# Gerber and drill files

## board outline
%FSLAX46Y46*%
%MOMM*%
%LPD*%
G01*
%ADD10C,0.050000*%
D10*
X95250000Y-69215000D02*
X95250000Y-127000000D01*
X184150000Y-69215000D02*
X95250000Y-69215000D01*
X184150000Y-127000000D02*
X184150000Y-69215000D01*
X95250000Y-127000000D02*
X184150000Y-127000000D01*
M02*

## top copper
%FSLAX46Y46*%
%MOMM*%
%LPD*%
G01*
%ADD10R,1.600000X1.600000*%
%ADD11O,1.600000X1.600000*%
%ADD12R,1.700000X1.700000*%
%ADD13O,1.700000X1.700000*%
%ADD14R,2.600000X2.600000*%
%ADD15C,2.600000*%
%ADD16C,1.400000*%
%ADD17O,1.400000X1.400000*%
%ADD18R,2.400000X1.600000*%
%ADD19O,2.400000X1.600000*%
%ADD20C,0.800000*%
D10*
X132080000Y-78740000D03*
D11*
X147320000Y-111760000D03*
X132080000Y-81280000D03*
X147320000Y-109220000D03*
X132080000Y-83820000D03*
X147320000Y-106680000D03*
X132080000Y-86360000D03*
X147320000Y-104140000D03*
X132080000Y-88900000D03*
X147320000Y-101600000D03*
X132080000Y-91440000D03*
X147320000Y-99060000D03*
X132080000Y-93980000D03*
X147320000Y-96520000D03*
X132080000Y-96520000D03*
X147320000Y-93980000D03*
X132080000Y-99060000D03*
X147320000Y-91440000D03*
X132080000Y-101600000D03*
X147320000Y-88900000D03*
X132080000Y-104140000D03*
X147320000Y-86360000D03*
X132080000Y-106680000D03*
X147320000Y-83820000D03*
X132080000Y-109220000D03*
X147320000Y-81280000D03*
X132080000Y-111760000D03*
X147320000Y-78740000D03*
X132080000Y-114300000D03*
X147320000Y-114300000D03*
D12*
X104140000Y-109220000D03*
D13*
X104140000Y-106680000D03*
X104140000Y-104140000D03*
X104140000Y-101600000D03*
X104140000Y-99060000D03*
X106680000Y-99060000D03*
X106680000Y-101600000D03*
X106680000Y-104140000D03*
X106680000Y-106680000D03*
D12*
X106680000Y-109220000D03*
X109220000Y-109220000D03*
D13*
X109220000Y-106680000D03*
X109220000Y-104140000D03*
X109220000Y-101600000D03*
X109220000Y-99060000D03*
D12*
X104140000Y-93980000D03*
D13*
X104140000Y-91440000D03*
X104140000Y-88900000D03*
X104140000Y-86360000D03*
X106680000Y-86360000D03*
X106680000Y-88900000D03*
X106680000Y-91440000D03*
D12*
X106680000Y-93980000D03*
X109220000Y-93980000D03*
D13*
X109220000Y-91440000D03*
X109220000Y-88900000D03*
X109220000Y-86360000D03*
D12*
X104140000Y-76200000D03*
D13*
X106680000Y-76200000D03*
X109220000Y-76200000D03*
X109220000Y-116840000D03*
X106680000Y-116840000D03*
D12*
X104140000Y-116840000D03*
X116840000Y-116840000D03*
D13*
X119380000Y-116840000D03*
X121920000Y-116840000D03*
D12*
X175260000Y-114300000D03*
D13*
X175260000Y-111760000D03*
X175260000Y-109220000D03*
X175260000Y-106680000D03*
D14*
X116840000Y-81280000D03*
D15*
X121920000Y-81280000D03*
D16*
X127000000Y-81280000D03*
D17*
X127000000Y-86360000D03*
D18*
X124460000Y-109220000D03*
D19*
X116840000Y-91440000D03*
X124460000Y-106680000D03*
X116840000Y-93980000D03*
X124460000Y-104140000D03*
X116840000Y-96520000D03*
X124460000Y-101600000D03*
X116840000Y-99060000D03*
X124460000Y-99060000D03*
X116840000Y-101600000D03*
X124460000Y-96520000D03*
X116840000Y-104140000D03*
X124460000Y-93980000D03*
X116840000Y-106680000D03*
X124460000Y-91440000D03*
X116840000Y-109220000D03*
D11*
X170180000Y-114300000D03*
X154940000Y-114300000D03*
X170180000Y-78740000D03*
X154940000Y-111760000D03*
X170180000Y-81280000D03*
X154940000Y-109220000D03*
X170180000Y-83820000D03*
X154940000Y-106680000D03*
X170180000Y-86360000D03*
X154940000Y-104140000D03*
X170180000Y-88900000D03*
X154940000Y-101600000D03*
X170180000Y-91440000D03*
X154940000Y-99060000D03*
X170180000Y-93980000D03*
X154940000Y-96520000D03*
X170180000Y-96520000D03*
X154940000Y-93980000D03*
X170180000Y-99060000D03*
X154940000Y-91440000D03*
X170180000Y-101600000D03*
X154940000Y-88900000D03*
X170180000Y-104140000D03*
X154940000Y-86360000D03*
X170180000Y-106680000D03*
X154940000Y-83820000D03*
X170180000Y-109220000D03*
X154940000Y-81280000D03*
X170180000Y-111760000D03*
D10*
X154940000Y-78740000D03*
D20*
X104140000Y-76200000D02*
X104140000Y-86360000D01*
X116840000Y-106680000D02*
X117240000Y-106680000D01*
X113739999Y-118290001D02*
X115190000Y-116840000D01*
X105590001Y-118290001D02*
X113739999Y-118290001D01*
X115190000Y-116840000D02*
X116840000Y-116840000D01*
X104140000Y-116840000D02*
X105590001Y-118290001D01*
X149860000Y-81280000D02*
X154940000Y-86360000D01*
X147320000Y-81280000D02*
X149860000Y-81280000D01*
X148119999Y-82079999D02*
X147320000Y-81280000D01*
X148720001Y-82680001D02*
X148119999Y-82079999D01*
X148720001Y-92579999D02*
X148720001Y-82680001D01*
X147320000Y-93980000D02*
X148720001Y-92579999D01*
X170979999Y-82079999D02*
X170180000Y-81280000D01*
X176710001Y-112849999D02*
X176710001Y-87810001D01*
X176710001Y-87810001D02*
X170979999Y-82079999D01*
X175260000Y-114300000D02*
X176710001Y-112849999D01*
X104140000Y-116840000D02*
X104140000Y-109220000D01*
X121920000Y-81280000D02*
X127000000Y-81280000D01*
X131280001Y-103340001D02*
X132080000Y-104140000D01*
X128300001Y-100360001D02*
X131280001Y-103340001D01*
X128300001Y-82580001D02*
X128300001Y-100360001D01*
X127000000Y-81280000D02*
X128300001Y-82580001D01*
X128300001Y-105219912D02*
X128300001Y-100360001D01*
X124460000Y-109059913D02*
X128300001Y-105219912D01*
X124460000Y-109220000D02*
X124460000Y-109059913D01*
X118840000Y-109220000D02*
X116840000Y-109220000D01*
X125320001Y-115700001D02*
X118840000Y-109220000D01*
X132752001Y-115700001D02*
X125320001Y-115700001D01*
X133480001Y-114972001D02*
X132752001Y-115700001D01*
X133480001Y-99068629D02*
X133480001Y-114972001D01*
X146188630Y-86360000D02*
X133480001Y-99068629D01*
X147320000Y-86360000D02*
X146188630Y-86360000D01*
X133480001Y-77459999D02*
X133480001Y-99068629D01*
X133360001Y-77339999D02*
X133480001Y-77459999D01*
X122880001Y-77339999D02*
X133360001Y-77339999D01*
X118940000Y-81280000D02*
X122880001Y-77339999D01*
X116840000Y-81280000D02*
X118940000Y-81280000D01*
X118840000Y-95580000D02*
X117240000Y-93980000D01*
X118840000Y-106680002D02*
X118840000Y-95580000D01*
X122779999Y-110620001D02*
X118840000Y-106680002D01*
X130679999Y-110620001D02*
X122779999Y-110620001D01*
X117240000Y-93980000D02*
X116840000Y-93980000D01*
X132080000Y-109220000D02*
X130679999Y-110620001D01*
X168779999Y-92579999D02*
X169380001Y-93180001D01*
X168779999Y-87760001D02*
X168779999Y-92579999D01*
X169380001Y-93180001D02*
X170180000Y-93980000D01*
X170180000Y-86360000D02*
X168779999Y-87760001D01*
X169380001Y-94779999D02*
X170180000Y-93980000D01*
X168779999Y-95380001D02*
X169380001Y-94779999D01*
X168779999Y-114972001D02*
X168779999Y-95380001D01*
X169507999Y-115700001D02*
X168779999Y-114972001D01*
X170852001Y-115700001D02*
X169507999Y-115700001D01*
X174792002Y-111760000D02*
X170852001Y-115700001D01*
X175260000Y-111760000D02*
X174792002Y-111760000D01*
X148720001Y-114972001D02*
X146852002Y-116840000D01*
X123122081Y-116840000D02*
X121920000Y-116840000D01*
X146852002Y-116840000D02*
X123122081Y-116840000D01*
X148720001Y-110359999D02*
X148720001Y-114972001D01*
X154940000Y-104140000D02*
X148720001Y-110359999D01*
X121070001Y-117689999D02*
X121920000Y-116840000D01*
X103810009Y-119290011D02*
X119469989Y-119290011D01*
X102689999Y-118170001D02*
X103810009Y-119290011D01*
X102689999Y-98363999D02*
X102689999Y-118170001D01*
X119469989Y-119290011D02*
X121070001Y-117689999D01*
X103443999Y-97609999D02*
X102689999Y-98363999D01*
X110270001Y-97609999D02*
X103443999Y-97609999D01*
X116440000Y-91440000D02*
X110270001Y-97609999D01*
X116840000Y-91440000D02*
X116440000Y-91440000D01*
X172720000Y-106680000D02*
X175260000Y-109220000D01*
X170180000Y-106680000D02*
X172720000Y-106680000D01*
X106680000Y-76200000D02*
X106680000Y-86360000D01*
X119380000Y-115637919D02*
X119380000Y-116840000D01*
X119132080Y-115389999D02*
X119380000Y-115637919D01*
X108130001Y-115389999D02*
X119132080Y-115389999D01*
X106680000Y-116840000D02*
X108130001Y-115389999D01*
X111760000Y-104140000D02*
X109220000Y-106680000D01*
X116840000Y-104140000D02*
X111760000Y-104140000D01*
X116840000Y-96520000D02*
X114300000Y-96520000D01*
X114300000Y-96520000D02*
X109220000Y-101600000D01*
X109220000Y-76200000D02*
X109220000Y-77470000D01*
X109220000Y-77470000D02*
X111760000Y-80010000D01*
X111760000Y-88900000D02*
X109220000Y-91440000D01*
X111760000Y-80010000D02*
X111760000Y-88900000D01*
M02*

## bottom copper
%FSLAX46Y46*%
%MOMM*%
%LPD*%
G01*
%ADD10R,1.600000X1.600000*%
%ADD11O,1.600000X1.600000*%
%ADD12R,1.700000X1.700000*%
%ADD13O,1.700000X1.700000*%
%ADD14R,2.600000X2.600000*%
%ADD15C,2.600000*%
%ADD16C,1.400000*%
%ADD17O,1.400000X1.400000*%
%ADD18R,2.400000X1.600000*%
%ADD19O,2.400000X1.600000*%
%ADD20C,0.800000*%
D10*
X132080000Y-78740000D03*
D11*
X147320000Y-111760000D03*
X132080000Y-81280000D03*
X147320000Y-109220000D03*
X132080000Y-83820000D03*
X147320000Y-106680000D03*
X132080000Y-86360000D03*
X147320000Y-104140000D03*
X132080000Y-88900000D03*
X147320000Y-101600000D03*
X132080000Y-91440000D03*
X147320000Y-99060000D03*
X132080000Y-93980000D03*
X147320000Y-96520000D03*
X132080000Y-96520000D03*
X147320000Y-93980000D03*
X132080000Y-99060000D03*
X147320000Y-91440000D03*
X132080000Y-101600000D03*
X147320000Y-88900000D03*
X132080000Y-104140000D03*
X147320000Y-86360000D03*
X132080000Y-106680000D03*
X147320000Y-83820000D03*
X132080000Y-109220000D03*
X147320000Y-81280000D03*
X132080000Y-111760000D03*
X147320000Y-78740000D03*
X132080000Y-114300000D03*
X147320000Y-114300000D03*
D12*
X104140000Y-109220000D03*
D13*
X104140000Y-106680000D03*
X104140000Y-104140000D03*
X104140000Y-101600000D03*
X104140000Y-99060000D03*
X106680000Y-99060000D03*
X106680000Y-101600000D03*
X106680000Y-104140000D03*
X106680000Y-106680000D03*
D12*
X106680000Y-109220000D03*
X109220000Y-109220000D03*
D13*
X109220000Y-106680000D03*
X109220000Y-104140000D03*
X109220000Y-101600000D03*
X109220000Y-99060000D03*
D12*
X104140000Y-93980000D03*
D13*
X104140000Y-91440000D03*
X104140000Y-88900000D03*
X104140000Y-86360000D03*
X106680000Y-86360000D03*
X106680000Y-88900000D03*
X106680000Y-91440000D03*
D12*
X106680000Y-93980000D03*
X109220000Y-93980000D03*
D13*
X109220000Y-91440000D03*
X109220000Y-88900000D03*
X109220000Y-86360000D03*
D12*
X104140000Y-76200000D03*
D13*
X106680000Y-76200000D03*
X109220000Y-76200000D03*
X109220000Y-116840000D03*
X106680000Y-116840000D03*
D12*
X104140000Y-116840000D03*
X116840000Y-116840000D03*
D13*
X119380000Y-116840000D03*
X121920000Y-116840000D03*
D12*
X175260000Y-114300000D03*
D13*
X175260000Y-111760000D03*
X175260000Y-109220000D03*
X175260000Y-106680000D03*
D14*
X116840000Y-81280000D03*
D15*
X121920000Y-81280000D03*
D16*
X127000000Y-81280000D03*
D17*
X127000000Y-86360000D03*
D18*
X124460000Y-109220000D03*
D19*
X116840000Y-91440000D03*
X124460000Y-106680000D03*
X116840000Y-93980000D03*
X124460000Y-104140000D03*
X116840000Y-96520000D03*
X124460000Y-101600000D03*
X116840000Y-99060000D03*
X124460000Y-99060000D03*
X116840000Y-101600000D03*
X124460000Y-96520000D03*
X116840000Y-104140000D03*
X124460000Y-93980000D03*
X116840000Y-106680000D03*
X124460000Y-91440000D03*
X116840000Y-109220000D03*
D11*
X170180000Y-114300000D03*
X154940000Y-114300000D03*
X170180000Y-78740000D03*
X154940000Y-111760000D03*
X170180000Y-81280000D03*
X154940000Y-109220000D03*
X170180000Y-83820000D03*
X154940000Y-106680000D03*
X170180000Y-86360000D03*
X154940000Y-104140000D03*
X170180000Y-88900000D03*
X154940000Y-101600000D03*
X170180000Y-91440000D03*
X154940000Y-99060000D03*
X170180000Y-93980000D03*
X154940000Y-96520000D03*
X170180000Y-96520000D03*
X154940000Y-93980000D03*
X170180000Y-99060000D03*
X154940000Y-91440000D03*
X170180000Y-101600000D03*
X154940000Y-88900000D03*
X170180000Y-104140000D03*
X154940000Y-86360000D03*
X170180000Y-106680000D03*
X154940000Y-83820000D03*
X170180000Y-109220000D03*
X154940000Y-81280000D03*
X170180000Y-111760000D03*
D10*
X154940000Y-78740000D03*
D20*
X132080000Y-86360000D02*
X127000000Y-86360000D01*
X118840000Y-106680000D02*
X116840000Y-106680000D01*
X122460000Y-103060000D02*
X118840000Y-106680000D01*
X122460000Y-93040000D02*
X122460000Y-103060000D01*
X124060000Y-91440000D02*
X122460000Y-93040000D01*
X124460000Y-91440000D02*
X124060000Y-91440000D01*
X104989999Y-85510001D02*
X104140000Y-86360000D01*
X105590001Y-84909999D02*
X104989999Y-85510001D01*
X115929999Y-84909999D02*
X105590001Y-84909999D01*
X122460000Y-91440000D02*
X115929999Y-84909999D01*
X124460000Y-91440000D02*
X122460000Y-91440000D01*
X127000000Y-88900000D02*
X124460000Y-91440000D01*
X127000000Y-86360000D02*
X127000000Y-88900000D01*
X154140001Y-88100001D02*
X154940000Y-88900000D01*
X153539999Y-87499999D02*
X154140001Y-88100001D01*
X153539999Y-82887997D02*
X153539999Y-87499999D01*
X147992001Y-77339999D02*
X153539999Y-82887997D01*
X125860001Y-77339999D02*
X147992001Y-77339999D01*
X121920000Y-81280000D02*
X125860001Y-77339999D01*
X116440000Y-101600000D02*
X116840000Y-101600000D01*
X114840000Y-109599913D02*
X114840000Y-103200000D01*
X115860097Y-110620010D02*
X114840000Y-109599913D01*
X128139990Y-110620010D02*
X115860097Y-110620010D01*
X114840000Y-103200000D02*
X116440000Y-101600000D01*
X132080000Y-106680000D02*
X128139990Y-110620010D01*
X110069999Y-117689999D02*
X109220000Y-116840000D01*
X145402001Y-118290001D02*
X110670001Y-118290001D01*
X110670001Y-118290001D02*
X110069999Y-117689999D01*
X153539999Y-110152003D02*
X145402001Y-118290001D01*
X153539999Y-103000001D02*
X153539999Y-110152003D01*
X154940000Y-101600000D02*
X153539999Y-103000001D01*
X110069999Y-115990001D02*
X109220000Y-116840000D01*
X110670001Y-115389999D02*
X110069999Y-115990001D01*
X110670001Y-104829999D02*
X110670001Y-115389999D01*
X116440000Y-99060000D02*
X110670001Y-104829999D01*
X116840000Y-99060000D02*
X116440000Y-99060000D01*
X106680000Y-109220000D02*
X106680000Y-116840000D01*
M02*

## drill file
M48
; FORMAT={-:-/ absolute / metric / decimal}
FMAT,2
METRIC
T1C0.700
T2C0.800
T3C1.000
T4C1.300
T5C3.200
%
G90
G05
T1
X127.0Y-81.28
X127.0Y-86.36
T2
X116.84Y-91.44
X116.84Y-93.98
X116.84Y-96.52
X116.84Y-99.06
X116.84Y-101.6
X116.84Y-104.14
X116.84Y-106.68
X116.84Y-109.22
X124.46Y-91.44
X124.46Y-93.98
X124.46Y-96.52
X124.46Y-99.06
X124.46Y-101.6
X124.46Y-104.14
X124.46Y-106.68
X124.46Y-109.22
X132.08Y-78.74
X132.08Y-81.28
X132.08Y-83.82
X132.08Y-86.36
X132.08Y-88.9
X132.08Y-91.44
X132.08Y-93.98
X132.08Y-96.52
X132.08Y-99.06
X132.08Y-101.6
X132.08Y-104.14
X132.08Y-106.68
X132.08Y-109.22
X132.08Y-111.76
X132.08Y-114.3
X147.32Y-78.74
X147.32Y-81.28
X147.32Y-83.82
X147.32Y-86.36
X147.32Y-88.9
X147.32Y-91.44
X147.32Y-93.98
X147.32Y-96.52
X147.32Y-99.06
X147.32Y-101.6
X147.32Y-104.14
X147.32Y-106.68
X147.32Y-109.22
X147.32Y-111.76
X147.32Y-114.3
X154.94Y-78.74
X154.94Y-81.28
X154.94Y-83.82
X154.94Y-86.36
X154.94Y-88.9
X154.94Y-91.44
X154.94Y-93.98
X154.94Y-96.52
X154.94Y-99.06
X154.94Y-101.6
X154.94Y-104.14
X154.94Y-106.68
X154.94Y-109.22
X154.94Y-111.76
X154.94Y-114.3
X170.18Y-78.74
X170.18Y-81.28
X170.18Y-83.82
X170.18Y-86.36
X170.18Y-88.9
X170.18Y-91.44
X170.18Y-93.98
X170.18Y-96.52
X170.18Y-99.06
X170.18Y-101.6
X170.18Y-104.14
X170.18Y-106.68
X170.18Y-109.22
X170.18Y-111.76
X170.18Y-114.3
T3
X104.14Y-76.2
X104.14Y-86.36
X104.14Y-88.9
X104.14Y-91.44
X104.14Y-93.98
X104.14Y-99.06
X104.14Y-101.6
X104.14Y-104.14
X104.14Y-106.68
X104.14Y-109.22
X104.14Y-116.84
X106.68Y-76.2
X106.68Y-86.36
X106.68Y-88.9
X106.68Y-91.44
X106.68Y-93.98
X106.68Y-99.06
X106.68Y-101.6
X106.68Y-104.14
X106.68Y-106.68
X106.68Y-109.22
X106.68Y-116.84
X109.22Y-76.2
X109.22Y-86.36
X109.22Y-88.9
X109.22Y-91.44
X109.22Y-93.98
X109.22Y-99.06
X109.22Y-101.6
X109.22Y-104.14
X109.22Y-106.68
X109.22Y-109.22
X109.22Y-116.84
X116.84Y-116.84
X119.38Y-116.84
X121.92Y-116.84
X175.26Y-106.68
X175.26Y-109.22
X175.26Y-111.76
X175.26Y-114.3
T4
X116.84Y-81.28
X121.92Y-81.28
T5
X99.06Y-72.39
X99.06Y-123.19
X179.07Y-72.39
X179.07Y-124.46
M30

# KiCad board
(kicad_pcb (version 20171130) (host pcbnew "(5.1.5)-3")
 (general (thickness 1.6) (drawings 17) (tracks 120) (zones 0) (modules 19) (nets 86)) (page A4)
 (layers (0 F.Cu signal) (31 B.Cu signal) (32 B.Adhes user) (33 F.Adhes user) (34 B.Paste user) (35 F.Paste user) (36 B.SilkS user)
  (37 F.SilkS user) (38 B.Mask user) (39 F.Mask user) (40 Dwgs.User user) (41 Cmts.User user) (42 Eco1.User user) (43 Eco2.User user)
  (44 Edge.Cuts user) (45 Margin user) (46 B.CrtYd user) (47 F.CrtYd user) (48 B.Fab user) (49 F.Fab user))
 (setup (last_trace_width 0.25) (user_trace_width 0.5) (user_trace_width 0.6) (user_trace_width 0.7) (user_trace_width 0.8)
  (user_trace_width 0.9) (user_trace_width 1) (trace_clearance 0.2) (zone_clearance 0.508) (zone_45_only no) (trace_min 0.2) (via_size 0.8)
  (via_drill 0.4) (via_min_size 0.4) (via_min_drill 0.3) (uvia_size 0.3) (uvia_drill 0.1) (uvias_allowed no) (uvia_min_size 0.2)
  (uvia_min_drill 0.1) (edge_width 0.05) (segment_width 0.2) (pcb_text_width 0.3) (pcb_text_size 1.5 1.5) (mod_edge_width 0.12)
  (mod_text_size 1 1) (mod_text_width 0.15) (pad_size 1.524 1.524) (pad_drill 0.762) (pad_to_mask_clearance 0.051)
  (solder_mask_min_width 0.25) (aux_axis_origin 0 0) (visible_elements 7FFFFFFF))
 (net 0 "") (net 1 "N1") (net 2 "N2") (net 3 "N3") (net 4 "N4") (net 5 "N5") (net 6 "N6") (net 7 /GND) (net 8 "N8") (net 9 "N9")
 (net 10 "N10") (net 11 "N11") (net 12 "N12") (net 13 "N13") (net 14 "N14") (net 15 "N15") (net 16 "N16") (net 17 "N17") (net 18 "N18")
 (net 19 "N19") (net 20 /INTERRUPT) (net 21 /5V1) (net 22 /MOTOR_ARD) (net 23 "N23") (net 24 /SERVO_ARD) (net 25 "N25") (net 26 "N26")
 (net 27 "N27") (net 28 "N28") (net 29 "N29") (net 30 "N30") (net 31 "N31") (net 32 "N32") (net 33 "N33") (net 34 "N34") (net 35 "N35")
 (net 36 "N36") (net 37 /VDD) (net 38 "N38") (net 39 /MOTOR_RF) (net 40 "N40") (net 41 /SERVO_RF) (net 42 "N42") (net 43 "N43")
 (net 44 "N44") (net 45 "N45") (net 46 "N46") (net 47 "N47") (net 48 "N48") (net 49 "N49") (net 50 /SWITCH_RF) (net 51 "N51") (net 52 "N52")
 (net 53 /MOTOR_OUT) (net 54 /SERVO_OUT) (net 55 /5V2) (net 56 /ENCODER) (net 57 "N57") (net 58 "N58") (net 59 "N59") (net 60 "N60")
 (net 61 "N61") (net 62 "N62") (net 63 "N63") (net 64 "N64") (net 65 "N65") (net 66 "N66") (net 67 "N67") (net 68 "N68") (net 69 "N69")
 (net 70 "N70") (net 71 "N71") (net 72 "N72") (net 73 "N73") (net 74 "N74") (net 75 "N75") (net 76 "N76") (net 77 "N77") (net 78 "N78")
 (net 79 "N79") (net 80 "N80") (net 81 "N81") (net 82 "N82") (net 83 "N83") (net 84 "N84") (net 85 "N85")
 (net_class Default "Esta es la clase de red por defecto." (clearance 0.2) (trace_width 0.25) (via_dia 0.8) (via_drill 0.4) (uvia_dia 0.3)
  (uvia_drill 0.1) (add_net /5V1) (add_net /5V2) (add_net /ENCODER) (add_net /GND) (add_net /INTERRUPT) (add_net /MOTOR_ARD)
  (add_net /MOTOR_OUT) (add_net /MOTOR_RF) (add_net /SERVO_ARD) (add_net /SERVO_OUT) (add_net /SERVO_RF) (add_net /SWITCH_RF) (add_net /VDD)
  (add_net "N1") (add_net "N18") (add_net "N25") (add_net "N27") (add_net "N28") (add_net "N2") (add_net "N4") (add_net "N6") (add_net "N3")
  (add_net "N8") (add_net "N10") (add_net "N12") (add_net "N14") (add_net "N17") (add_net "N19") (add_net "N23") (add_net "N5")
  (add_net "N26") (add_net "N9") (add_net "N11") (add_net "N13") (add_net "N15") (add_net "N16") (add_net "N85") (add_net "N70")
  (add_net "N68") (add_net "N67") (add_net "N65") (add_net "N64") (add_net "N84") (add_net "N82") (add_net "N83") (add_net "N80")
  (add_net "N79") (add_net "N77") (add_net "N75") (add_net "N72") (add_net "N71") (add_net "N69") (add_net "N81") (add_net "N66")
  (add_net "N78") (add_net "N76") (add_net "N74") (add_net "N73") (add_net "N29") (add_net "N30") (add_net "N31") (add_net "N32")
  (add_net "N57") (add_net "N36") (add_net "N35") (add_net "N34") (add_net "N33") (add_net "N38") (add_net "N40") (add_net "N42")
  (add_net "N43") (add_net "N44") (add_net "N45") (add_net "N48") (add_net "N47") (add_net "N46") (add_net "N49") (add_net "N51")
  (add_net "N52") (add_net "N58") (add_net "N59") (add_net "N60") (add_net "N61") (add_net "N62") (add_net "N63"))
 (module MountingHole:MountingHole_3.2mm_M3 (layer F.Cu) (at 99.06 123.19)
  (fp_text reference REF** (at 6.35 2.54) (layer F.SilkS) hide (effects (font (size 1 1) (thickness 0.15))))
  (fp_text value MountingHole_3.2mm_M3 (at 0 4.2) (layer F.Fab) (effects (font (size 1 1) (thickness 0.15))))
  (pad 1 np_thru_hole circle (at 0 0) (size 3.2 3.2) (drill 3.2) (layers *.Cu *.Mask)))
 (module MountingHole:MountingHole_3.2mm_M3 (layer F.Cu) (at 99.06 72.39)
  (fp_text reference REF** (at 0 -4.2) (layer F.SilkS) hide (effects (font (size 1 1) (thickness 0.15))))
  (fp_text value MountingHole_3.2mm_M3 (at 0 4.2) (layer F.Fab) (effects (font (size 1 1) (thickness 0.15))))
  (pad 1 np_thru_hole circle (at 0 0) (size 3.2 3.2) (drill 3.2) (layers *.Cu *.Mask)))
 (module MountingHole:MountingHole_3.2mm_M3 (layer F.Cu) (at 179.07 72.39)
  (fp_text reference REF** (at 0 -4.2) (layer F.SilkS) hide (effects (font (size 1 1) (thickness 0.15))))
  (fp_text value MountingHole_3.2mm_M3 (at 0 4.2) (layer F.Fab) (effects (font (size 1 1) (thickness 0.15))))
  (pad 1 np_thru_hole circle (at 0 0) (size 3.2 3.2) (drill 3.2) (layers *.Cu *.Mask)))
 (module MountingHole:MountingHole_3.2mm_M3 (layer F.Cu) (at 179.07 124.46)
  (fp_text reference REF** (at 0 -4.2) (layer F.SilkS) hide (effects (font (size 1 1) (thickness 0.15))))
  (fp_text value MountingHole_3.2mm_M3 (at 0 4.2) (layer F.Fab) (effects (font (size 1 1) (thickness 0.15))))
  (pad 1 np_thru_hole circle (at 0 0) (size 3.2 3.2) (drill 3.2) (layers *.Cu *.Mask)))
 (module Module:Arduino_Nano (layer F.Cu) (at 132.08 78.74)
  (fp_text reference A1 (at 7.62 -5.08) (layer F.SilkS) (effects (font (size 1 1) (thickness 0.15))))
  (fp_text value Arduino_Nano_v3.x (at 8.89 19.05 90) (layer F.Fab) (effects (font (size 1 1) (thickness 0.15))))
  (pad 1 thru_hole rect (at 0 0) (size 1.6 1.6) (drill 0.8) (layers *.Cu *.Mask) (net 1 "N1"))
  (pad 17 thru_hole oval (at 15.24 33.02) (size 1.6 1.6) (drill 0.8) (layers *.Cu *.Mask) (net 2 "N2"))
  (pad 2 thru_hole oval (at 0 2.54) (size 1.6 1.6) (drill 0.8) (layers *.Cu *.Mask) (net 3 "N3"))
  (pad 18 thru_hole oval (at 15.24 30.48) (size 1.6 1.6) (drill 0.8) (layers *.Cu *.Mask) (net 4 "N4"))
  (pad 3 thru_hole oval (at 0 5.08) (size 1.6 1.6) (drill 0.8) (layers *.Cu *.Mask) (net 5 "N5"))
  (pad 19 thru_hole oval (at 15.24 27.94) (size 1.6 1.6) (drill 0.8) (layers *.Cu *.Mask) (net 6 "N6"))
  (pad 4 thru_hole oval (at 0 7.62) (size 1.6 1.6) (drill 0.8) (layers *.Cu *.Mask) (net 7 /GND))
  (pad 20 thru_hole oval (at 15.24 25.4) (size 1.6 1.6) (drill 0.8) (layers *.Cu *.Mask) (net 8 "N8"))
  (pad 5 thru_hole oval (at 0 10.16) (size 1.6 1.6) (drill 0.8) (layers *.Cu *.Mask) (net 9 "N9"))
  (pad 21 thru_hole oval (at 15.24 22.86) (size 1.6 1.6) (drill 0.8) (layers *.Cu *.Mask) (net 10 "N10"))
  (pad 6 thru_hole oval (at 0 12.7) (size 1.6 1.6) (drill 0.8) (layers *.Cu *.Mask) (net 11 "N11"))
  (pad 22 thru_hole oval (at 15.24 20.32) (size 1.6 1.6) (drill 0.8) (layers *.Cu *.Mask) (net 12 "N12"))
  (pad 7 thru_hole oval (at 0 15.24) (size 1.6 1.6) (drill 0.8) (layers *.Cu *.Mask) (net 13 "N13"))
  (pad 23 thru_hole oval (at 15.24 17.78) (size 1.6 1.6) (drill 0.8) (layers *.Cu *.Mask) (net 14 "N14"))
  (pad 8 thru_hole oval (at 0 17.78) (size 1.6 1.6) (drill 0.8) (layers *.Cu *.Mask) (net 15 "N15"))
  (pad 24 thru_hole oval (at 15.24 15.24) (size 1.6 1.6) (drill 0.8) (layers *.Cu *.Mask) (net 7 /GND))
  (pad 9 thru_hole oval (at 0 20.32) (size 1.6 1.6) (drill 0.8) (layers *.Cu *.Mask) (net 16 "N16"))
  (pad 25 thru_hole oval (at 15.24 12.7) (size 1.6 1.6) (drill 0.8) (layers *.Cu *.Mask) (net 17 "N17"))
  (pad 10 thru_hole oval (at 0 22.86) (size 1.6 1.6) (drill 0.8) (layers *.Cu *.Mask) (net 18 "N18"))
  (pad 26 thru_hole oval (at 15.24 10.16) (size 1.6 1.6) (drill 0.8) (layers *.Cu *.Mask) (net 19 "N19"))
  (pad 11 thru_hole oval (at 0 25.4) (size 1.6 1.6) (drill 0.8) (layers *.Cu *.Mask) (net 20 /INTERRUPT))
  (pad 27 thru_hole oval (at 15.24 7.62) (size 1.6 1.6) (drill 0.8) (layers *.Cu *.Mask) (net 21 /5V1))
  (pad 12 thru_hole oval (at 0 27.94) (size 1.6 1.6) (drill 0.8) (layers *.Cu *.Mask) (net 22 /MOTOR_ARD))
  (pad 28 thru_hole oval (at 15.24 5.08) (size 1.6 1.6) (drill 0.8) (layers *.Cu *.Mask) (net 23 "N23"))
  (pad 13 thru_hole oval (at 0 30.48) (size 1.6 1.6) (drill 0.8) (layers *.Cu *.Mask) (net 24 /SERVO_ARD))
  (pad 29 thru_hole oval (at 15.24 2.54) (size 1.6 1.6) (drill 0.8) (layers *.Cu *.Mask) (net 7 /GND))
  (pad 14 thru_hole oval (at 0 33.02) (size 1.6 1.6) (drill 0.8) (layers *.Cu *.Mask) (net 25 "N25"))
  (pad 30 thru_hole oval (at 15.24 0) (size 1.6 1.6) (drill 0.8) (layers *.Cu *.Mask) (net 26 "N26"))
  (pad 15 thru_hole oval (at 0 35.56) (size 1.6 1.6) (drill 0.8) (layers *.Cu *.Mask) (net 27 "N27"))
  (pad 16 thru_hole oval (at 15.24 35.56) (size 1.6 1.6) (drill 0.8) (layers *.Cu *.Mask) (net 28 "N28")))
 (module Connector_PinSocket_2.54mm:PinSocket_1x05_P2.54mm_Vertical (layer F.Cu) (at 104.14 109.22 180)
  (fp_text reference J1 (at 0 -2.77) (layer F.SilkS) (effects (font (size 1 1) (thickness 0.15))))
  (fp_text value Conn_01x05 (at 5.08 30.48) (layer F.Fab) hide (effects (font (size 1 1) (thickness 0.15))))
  (pad 1 thru_hole rect (at 0 0 180) (size 1.7 1.7) (drill 1) (layers *.Cu *.Mask) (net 7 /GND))
  (pad 2 thru_hole oval (at 0 2.54 180) (size 1.7 1.7) (drill 1) (layers *.Cu *.Mask) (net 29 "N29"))
  (pad 3 thru_hole oval (at 0 5.08 180) (size 1.7 1.7) (drill 1) (layers *.Cu *.Mask) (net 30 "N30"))
  (pad 4 thru_hole oval (at 0 7.62 180) (size 1.7 1.7) (drill 1) (layers *.Cu *.Mask) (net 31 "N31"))
  (pad 5 thru_hole oval (at 0 10.16 180) (size 1.7 1.7) (drill 1) (layers *.Cu *.Mask) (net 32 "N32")))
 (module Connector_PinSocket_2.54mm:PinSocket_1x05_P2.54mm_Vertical (layer F.Cu) (at 106.68 109.22 180)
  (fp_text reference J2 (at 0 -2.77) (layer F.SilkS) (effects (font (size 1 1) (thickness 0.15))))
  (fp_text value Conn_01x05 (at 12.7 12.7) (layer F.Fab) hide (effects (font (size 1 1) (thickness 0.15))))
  (pad 5 thru_hole oval (at 0 10.16 180) (size 1.7 1.7) (drill 1) (layers *.Cu *.Mask) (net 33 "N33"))
  (pad 4 thru_hole oval (at 0 7.62 180) (size 1.7 1.7) (drill 1) (layers *.Cu *.Mask) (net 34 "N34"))
  (pad 3 thru_hole oval (at 0 5.08 180) (size 1.7 1.7) (drill 1) (layers *.Cu *.Mask) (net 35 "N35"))
  (pad 2 thru_hole oval (at 0 2.54 180) (size 1.7 1.7) (drill 1) (layers *.Cu *.Mask) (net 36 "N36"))
  (pad 1 thru_hole rect (at 0 0 180) (size 1.7 1.7) (drill 1) (layers *.Cu *.Mask) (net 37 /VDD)))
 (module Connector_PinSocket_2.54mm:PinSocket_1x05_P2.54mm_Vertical (layer F.Cu) (at 109.22 109.22 180)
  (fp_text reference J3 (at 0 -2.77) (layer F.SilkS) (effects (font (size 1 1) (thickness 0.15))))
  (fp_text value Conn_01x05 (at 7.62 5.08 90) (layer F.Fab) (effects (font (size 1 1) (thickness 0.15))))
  (pad 1 thru_hole rect (at 0 0 180) (size 1.7 1.7) (drill 1) (layers *.Cu *.Mask) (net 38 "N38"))
  (pad 2 thru_hole oval (at 0 2.54 180) (size 1.7 1.7) (drill 1) (layers *.Cu *.Mask) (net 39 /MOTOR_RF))
  (pad 3 thru_hole oval (at 0 5.08 180) (size 1.7 1.7) (drill 1) (layers *.Cu *.Mask) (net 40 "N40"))
  (pad 4 thru_hole oval (at 0 7.62 180) (size 1.7 1.7) (drill 1) (layers *.Cu *.Mask) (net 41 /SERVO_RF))
  (pad 5 thru_hole oval (at 0 10.16 180) (size 1.7 1.7) (drill 1) (layers *.Cu *.Mask) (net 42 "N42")))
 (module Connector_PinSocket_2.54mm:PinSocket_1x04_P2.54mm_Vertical (layer F.Cu) (at 104.14 93.98 180)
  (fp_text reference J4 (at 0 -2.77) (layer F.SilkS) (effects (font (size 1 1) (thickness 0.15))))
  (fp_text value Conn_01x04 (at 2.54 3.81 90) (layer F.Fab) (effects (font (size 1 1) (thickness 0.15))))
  (pad 1 thru_hole rect (at 0 0 180) (size 1.7 1.7) (drill 1) (layers *.Cu *.Mask) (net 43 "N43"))
  (pad 2 thru_hole oval (at 0 2.54 180) (size 1.7 1.7) (drill 1) (layers *.Cu *.Mask) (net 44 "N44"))
  (pad 3 thru_hole oval (at 0 5.08 180) (size 1.7 1.7) (drill 1) (layers *.Cu *.Mask) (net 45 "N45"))
  (pad 4 thru_hole oval (at 0 7.62 180) (size 1.7 1.7) (drill 1) (layers *.Cu *.Mask) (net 7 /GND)))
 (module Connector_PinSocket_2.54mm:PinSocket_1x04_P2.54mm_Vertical (layer F.Cu) (at 106.68 93.98 180)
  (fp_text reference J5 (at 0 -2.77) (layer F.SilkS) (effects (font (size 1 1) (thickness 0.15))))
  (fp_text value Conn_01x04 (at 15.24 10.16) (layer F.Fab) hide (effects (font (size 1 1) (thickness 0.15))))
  (pad 4 thru_hole oval (at 0 7.62 180) (size 1.7 1.7) (drill 1) (layers *.Cu *.Mask) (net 37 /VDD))
  (pad 3 thru_hole oval (at 0 5.08 180) (size 1.7 1.7) (drill 1) (layers *.Cu *.Mask) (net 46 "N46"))
  (pad 2 thru_hole oval (at 0 2.54 180) (size 1.7 1.7) (drill 1) (layers *.Cu *.Mask) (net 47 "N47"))
  (pad 1 thru_hole rect (at 0 0 180) (size 1.7 1.7) (drill 1) (layers *.Cu *.Mask) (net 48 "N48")))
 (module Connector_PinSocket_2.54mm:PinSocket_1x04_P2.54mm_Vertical (layer F.Cu) (at 109.22 93.98 180)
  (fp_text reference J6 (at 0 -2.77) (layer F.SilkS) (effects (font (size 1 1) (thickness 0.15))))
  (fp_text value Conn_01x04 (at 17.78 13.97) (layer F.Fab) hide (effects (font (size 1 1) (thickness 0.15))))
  (pad 1 thru_hole rect (at 0 0 180) (size 1.7 1.7) (drill 1) (layers *.Cu *.Mask) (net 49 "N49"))
  (pad 2 thru_hole oval (at 0 2.54 180) (size 1.7 1.7) (drill 1) (layers *.Cu *.Mask) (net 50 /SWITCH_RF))
  (pad 3 thru_hole oval (at 0 5.08 180) (size 1.7 1.7) (drill 1) (layers *.Cu *.Mask) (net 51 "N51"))
  (pad 4 thru_hole oval (at 0 7.62 180) (size 1.7 1.7) (drill 1) (layers *.Cu *.Mask) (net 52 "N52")))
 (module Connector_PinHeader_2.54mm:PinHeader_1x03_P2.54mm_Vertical (layer F.Cu) (at 104.14 76.2 90)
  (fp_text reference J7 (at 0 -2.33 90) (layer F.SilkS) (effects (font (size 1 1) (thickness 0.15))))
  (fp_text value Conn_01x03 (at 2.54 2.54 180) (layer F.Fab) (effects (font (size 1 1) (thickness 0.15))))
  (pad 1 thru_hole rect (at 0 0 90) (size 1.7 1.7) (drill 1) (layers *.Cu *.Mask) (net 7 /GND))
  (pad 2 thru_hole oval (at 0 2.54 90) (size 1.7 1.7) (drill 1) (layers *.Cu *.Mask) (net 37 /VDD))
  (pad 3 thru_hole oval (at 0 5.08 90) (size 1.7 1.7) (drill 1) (layers *.Cu *.Mask) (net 50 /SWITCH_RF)))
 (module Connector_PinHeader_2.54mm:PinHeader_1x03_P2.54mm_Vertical (layer F.Cu) (at 104.14 116.84 90)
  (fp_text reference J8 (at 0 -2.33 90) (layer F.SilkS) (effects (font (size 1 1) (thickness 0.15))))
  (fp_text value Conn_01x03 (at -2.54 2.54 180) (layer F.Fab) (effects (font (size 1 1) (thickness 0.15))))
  (pad 3 thru_hole oval (at 0 5.08 90) (size 1.7 1.7) (drill 1) (layers *.Cu *.Mask) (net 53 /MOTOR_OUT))
  (pad 2 thru_hole oval (at 0 2.54 90) (size 1.7 1.7) (drill 1) (layers *.Cu *.Mask) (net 37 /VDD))
  (pad 1 thru_hole rect (at 0 0 90) (size 1.7 1.7) (drill 1) (layers *.Cu *.Mask) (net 7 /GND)))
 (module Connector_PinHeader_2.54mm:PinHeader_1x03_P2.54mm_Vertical (layer F.Cu) (at 116.84 116.84 90)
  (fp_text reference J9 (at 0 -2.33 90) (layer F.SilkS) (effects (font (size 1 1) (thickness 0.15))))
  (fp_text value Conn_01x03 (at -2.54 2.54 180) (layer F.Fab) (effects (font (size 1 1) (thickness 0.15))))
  (pad 1 thru_hole rect (at 0 0 90) (size 1.7 1.7) (drill 1) (layers *.Cu *.Mask) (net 7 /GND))
  (pad 2 thru_hole oval (at 0 2.54 90) (size 1.7 1.7) (drill 1) (layers *.Cu *.Mask) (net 37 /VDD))
  (pad 3 thru_hole oval (at 0 5.08 90) (size 1.7 1.7) (drill 1) (layers *.Cu *.Mask) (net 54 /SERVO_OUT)))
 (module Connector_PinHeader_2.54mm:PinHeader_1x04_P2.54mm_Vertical (layer F.Cu) (at 175.26 114.3 180)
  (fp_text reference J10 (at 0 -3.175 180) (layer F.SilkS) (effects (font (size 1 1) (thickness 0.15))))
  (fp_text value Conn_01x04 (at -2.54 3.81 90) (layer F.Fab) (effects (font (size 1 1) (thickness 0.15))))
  (pad 1 thru_hole rect (at 0 0 180) (size 1.7 1.7) (drill 1) (layers *.Cu *.Mask) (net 7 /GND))
  (pad 2 thru_hole oval (at 0 2.54 180) (size 1.7 1.7) (drill 1) (layers *.Cu *.Mask) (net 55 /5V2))
  (pad 3 thru_hole oval (at 0 5.08 180) (size 1.7 1.7) (drill 1) (layers *.Cu *.Mask) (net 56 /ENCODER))
  (pad 4 thru_hole oval (at 0 7.62 180) (size 1.7 1.7) (drill 1) (layers *.Cu *.Mask) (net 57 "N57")))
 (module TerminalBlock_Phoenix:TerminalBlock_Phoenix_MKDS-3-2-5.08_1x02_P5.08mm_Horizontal (layer F.Cu) (at 116.84 81.28)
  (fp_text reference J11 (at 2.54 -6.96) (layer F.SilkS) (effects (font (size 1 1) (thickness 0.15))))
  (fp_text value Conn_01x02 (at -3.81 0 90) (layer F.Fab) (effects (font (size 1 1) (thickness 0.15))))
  (pad 1 thru_hole rect (at 0 0) (size 2.6 2.6) (drill 1.3) (layers *.Cu *.Mask) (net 21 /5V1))
  (pad 2 thru_hole circle (at 5.08 0) (size 2.6 2.6) (drill 1.3) (layers *.Cu *.Mask) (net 20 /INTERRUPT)))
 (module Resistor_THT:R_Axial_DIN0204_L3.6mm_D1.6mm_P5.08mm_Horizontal (layer F.Cu) (at 127 81.28 270)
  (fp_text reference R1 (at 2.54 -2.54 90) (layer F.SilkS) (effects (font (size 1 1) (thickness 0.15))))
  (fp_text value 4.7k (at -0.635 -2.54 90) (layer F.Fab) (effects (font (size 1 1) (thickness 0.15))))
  (pad 1 thru_hole circle (at 0 0 270) (size 1.4 1.4) (drill 0.7) (layers *.Cu *.Mask) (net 20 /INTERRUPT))
  (pad 2 thru_hole oval (at 5.08 0 270) (size 1.4 1.4) (drill 0.7) (layers *.Cu *.Mask) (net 7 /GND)))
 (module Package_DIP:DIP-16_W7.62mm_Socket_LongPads (layer F.Cu) (at 124.46 109.22 180)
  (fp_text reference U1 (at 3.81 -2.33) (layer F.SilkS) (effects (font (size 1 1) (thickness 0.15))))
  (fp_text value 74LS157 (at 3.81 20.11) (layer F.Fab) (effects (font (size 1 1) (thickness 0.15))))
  (pad 1 thru_hole rect (at 0 0 180) (size 2.4 1.6) (drill 0.8) (layers *.Cu *.Mask) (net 20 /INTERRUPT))
  (pad 9 thru_hole oval (at 7.62 17.78 180) (size 2.4 1.6) (drill 0.8) (layers *.Cu *.Mask) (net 54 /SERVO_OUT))
  (pad 2 thru_hole oval (at 0 2.54 180) (size 2.4 1.6) (drill 0.8) (layers *.Cu *.Mask) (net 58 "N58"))
  (pad 10 thru_hole oval (at 7.62 15.24 180) (size 2.4 1.6) (drill 0.8) (layers *.Cu *.Mask) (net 24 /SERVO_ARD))
  (pad 3 thru_hole oval (at 0 5.08 180) (size 2.4 1.6) (drill 0.8) (layers *.Cu *.Mask) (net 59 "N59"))
  (pad 11 thru_hole oval (at 7.62 12.7 180) (size 2.4 1.6) (drill 0.8) (layers *.Cu *.Mask) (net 41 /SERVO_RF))
  (pad 4 thru_hole oval (at 0 7.62 180) (size 2.4 1.6) (drill 0.8) (layers *.Cu *.Mask) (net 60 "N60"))
  (pad 12 thru_hole oval (at 7.62 10.16 180) (size 2.4 1.6) (drill 0.8) (layers *.Cu *.Mask) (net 53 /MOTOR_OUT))
  (pad 5 thru_hole oval (at 0 10.16 180) (size 2.4 1.6) (drill 0.8) (layers *.Cu *.Mask) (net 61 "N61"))
  (pad 13 thru_hole oval (at 7.62 7.62 180) (size 2.4 1.6) (drill 0.8) (layers *.Cu *.Mask) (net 22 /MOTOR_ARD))
  (pad 6 thru_hole oval (at 0 12.7 180) (size 2.4 1.6) (drill 0.8) (layers *.Cu *.Mask) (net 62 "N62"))
  (pad 14 thru_hole oval (at 7.62 5.08 180) (size 2.4 1.6) (drill 0.8) (layers *.Cu *.Mask) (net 39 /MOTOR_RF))
  (pad 7 thru_hole oval (at 0 15.24 180) (size 2.4 1.6) (drill 0.8) (layers *.Cu *.Mask) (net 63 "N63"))
  (pad 15 thru_hole oval (at 7.62 2.54 180) (size 2.4 1.6) (drill 0.8) (layers *.Cu *.Mask) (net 7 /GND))
  (pad 8 thru_hole oval (at 0 17.78 180) (size 2.4 1.6) (drill 0.8) (layers *.Cu *.Mask) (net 7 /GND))
  (pad 16 thru_hole oval (at 7.62 0 180) (size 2.4 1.6) (drill 0.8) (layers *.Cu *.Mask) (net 21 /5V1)))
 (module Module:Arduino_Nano (layer F.Cu) (at 154.94 78.74)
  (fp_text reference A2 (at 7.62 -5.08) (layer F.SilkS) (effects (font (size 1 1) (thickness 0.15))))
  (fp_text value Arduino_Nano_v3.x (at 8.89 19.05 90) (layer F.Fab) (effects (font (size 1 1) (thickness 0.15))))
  (pad 16 thru_hole oval (at 15.24 35.56) (size 1.6 1.6) (drill 0.8) (layers *.Cu *.Mask) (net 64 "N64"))
  (pad 15 thru_hole oval (at 0 35.56) (size 1.6 1.6) (drill 0.8) (layers *.Cu *.Mask) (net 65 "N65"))
  (pad 30 thru_hole oval (at 15.24 0) (size 1.6 1.6) (drill 0.8) (layers *.Cu *.Mask) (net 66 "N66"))
  (pad 14 thru_hole oval (at 0 33.02) (size 1.6 1.6) (drill 0.8) (layers *.Cu *.Mask) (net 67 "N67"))
  (pad 29 thru_hole oval (at 15.24 2.54) (size 1.6 1.6) (drill 0.8) (layers *.Cu *.Mask) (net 7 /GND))
  (pad 13 thru_hole oval (at 0 30.48) (size 1.6 1.6) (drill 0.8) (layers *.Cu *.Mask) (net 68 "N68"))
  (pad 28 thru_hole oval (at 15.24 5.08) (size 1.6 1.6) (drill 0.8) (layers *.Cu *.Mask) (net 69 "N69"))
  (pad 12 thru_hole oval (at 0 27.94) (size 1.6 1.6) (drill 0.8) (layers *.Cu *.Mask) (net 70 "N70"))
  (pad 27 thru_hole oval (at 15.24 7.62) (size 1.6 1.6) (drill 0.8) (layers *.Cu *.Mask) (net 55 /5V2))
  (pad 11 thru_hole oval (at 0 25.4) (size 1.6 1.6) (drill 0.8) (layers *.Cu *.Mask) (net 54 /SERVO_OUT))
  (pad 26 thru_hole oval (at 15.24 10.16) (size 1.6 1.6) (drill 0.8) (layers *.Cu *.Mask) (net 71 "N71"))
  (pad 10 thru_hole oval (at 0 22.86) (size 1.6 1.6) (drill 0.8) (layers *.Cu *.Mask) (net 53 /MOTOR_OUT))
  (pad 25 thru_hole oval (at 15.24 12.7) (size 1.6 1.6) (drill 0.8) (layers *.Cu *.Mask) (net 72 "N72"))
  (pad 9 thru_hole oval (at 0 20.32) (size 1.6 1.6) (drill 0.8) (layers *.Cu *.Mask) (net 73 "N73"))
  (pad 24 thru_hole oval (at 15.24 15.24) (size 1.6 1.6) (drill 0.8) (layers *.Cu *.Mask) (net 55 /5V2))
  (pad 8 thru_hole oval (at 0 17.78) (size 1.6 1.6) (drill 0.8) (layers *.Cu *.Mask) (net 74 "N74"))
  (pad 23 thru_hole oval (at 15.24 17.78) (size 1.6 1.6) (drill 0.8) (layers *.Cu *.Mask) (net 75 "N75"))
  (pad 7 thru_hole oval (at 0 15.24) (size 1.6 1.6) (drill 0.8) (layers *.Cu *.Mask) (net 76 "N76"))
  (pad 22 thru_hole oval (at 15.24 20.32) (size 1.6 1.6) (drill 0.8) (layers *.Cu *.Mask) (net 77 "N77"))
  (pad 6 thru_hole oval (at 0 12.7) (size 1.6 1.6) (drill 0.8) (layers *.Cu *.Mask) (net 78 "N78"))
  (pad 21 thru_hole oval (at 15.24 22.86) (size 1.6 1.6) (drill 0.8) (layers *.Cu *.Mask) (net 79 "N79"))
  (pad 5 thru_hole oval (at 0 10.16) (size 1.6 1.6) (drill 0.8) (layers *.Cu *.Mask) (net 20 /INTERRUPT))
  (pad 20 thru_hole oval (at 15.24 25.4) (size 1.6 1.6) (drill 0.8) (layers *.Cu *.Mask) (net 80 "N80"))
  (pad 4 thru_hole oval (at 0 7.62) (size 1.6 1.6) (drill 0.8) (layers *.Cu *.Mask) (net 7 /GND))
  (pad 19 thru_hole oval (at 15.24 27.94) (size 1.6 1.6) (drill 0.8) (layers *.Cu *.Mask) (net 56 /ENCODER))
  (pad 3 thru_hole oval (at 0 5.08) (size 1.6 1.6) (drill 0.8) (layers *.Cu *.Mask) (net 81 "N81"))
  (pad 18 thru_hole oval (at 15.24 30.48) (size 1.6 1.6) (drill 0.8) (layers *.Cu *.Mask) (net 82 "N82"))
  (pad 2 thru_hole oval (at 0 2.54) (size 1.6 1.6) (drill 0.8) (layers *.Cu *.Mask) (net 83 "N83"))
  (pad 17 thru_hole oval (at 15.24 33.02) (size 1.6 1.6) (drill 0.8) (layers *.Cu *.Mask) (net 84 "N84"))
  (pad 1 thru_hole rect (at 0 0) (size 1.6 1.6) (drill 0.8) (layers *.Cu *.Mask) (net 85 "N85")))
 (gr_line (start 95.25 69.215) (end 95.25 127) (layer Edge.Cuts) (width 0.05))
 (gr_line (start 184.15 69.215) (end 95.25 69.215) (layer Edge.Cuts) (width 0.05))
 (gr_line (start 184.15 127) (end 184.15 69.215) (layer Edge.Cuts) (width 0.05))
 (gr_line (start 95.25 127) (end 184.15 127) (layer Edge.Cuts) (width 0.05))
 (segment (start 104.14 76.2) (end 104.14 86.36) (width 0.8) (layer F.Cu) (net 7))
 (segment (start 116.84 106.68) (end 117.24 106.68) (width 0.8) (layer F.Cu) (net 7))
 (segment (start 113.739999 118.290001) (end 115.19 116.84) (width 0.8) (layer F.Cu) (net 7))
 (segment (start 105.590001 118.290001) (end 113.739999 118.290001) (width 0.8) (layer F.Cu) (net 7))
 (segment (start 115.19 116.84) (end 116.84 116.84) (width 0.8) (layer F.Cu) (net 7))
 (segment (start 104.14 116.84) (end 105.590001 118.290001) (width 0.8) (layer F.Cu) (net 7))
 (segment (start 132.08 86.36) (end 127 86.36) (width 0.8) (layer B.Cu) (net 7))
 (segment (start 118.84 106.68) (end 116.84 106.68) (width 0.8) (layer B.Cu) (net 7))
 (segment (start 122.46 103.06) (end 118.84 106.68) (width 0.8) (layer B.Cu) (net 7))
 (segment (start 122.46 93.04) (end 122.46 103.06) (width 0.8) (layer B.Cu) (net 7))
 (segment (start 124.06 91.44) (end 122.46 93.04) (width 0.8) (layer B.Cu) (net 7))
 (segment (start 124.46 91.44) (end 124.06 91.44) (width 0.8) (layer B.Cu) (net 7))
 (segment (start 149.86 81.28) (end 154.94 86.36) (width 0.8) (layer F.Cu) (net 7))
 (segment (start 147.32 81.28) (end 149.86 81.28) (width 0.8) (layer F.Cu) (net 7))
 (segment (start 148.119999 82.079999) (end 147.32 81.28) (width 0.8) (layer F.Cu) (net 7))
 (segment (start 148.720001 82.680001) (end 148.119999 82.079999) (width 0.8) (layer F.Cu) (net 7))
 (segment (start 148.720001 92.579999) (end 148.720001 82.680001) (width 0.8) (layer F.Cu) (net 7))
 (segment (start 147.32 93.98) (end 148.720001 92.579999) (width 0.8) (layer F.Cu) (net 7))
 (segment (start 170.979999 82.079999) (end 170.18 81.28) (width 0.8) (layer F.Cu) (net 7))
 (segment (start 176.710001 112.849999) (end 176.710001 87.810001) (width 0.8) (layer F.Cu) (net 7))
 (segment (start 176.710001 87.810001) (end 170.979999 82.079999) (width 0.8) (layer F.Cu) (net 7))
 (segment (start 175.26 114.3) (end 176.710001 112.849999) (width 0.8) (layer F.Cu) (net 7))
 (segment (start 104.14 116.84) (end 104.14 109.22) (width 0.8) (layer F.Cu) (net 7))
 (segment (start 104.989999 85.510001) (end 104.14 86.36) (width 0.8) (layer B.Cu) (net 7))
 (segment (start 105.590001 84.909999) (end 104.989999 85.510001) (width 0.8) (layer B.Cu) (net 7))
 (segment (start 115.929999 84.909999) (end 105.590001 84.909999) (width 0.8) (layer B.Cu) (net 7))
 (segment (start 122.46 91.44) (end 115.929999 84.909999) (width 0.8) (layer B.Cu) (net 7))
 (segment (start 124.46 91.44) (end 122.46 91.44) (width 0.8) (layer B.Cu) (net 7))
 (segment (start 127 88.9) (end 124.46 91.44) (width 0.8) (layer B.Cu) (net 7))
 (segment (start 127 86.36) (end 127 88.9) (width 0.8) (layer B.Cu) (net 7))
 (segment (start 121.92 81.28) (end 127 81.28) (width 0.8) (layer F.Cu) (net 20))
 (segment (start 131.280001 103.340001) (end 132.08 104.14) (width 0.8) (layer F.Cu) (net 20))
 (segment (start 128.300001 100.360001) (end 131.280001 103.340001) (width 0.8) (layer F.Cu) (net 20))
 (segment (start 128.300001 82.580001) (end 128.300001 100.360001) (width 0.8) (layer F.Cu) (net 20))
 (segment (start 127 81.28) (end 128.300001 82.580001) (width 0.8) (layer F.Cu) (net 20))
 (segment (start 154.140001 88.100001) (end 154.94 88.9) (width 0.8) (layer B.Cu) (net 20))
 (segment (start 153.539999 87.499999) (end 154.140001 88.100001) (width 0.8) (layer B.Cu) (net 20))
 (segment (start 153.539999 82.887997) (end 153.539999 87.499999) (width 0.8) (layer B.Cu) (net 20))
 (segment (start 147.992001 77.339999) (end 153.539999 82.887997) (width 0.8) (layer B.Cu) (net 20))
 (segment (start 125.860001 77.339999) (end 147.992001 77.339999) (width 0.8) (layer B.Cu) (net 20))
 (segment (start 121.92 81.28) (end 125.860001 77.339999) (width 0.8) (layer B.Cu) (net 20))
 (segment (start 128.300001 105.219912) (end 128.300001 100.360001) (width 0.8) (layer F.Cu) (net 20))
 (segment (start 124.46 109.059913) (end 128.300001 105.219912) (width 0.8) (layer F.Cu) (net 20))
 (segment (start 124.46 109.22) (end 124.46 109.059913) (width 0.8) (layer F.Cu) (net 20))
 (segment (start 118.84 109.22) (end 116.84 109.22) (width 0.8) (layer F.Cu) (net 21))
 (segment (start 125.320001 115.700001) (end 118.84 109.22) (width 0.8) (layer F.Cu) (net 21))
 (segment (start 132.752001 115.700001) (end 125.320001 115.700001) (width 0.8) (layer F.Cu) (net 21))
 (segment (start 133.480001 114.972001) (end 132.752001 115.700001) (width 0.8) (layer F.Cu) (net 21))
 (segment (start 133.480001 99.068629) (end 133.480001 114.972001) (width 0.8) (layer F.Cu) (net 21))
 (segment (start 146.18863 86.36) (end 133.480001 99.068629) (width 0.8) (layer F.Cu) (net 21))
 (segment (start 147.32 86.36) (end 146.18863 86.36) (width 0.8) (layer F.Cu) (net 21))
 (segment (start 133.480001 77.459999) (end 133.480001 99.068629) (width 0.8) (layer F.Cu) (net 21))
 (segment (start 133.360001 77.339999) (end 133.480001 77.459999) (width 0.8) (layer F.Cu) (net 21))
 (segment (start 122.880001 77.339999) (end 133.360001 77.339999) (width 0.8) (layer F.Cu) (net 21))
 (segment (start 118.94 81.28) (end 122.880001 77.339999) (width 0.8) (layer F.Cu) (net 21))
 (segment (start 116.84 81.28) (end 118.94 81.28) (width 0.8) (layer F.Cu) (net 21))
 (segment (start 116.44 101.6) (end 116.84 101.6) (width 0.8) (layer B.Cu) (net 22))
 (segment (start 114.84 109.599913) (end 114.84 103.2) (width 0.8) (layer B.Cu) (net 22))
 (segment (start 115.860097 110.62001) (end 114.84 109.599913) (width 0.8) (layer B.Cu) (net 22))
 (segment (start 128.13999 110.62001) (end 115.860097 110.62001) (width 0.8) (layer B.Cu) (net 22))
 (segment (start 114.84 103.2) (end 116.44 101.6) (width 0.8) (layer B.Cu) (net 22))
 (segment (start 132.08 106.68) (end 128.13999 110.62001) (width 0.8) (layer B.Cu) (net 22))
 (segment (start 118.84 95.58) (end 117.24 93.98) (width 0.8) (layer F.Cu) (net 24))
 (segment (start 118.84 106.680002) (end 118.84 95.58) (width 0.8) (layer F.Cu) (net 24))
 (segment (start 122.779999 110.620001) (end 118.84 106.680002) (width 0.8) (layer F.Cu) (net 24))
 (segment (start 130.679999 110.620001) (end 122.779999 110.620001) (width 0.8) (layer F.Cu) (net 24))
 (segment (start 117.24 93.98) (end 116.84 93.98) (width 0.8) (layer F.Cu) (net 24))
 (segment (start 132.08 109.22) (end 130.679999 110.620001) (width 0.8) (layer F.Cu) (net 24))
 (segment (start 168.779999 92.579999) (end 169.380001 93.180001) (width 0.8) (layer F.Cu) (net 55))
 (segment (start 168.779999 87.760001) (end 168.779999 92.579999) (width 0.8) (layer F.Cu) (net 55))
 (segment (start 169.380001 93.180001) (end 170.18 93.98) (width 0.8) (layer F.Cu) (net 55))
 (segment (start 170.18 86.36) (end 168.779999 87.760001) (width 0.8) (layer F.Cu) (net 55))
 (segment (start 169.380001 94.779999) (end 170.18 93.98) (width 0.8) (layer F.Cu) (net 55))
 (segment (start 168.779999 95.380001) (end 169.380001 94.779999) (width 0.8) (layer F.Cu) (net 55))
 (segment (start 168.779999 114.972001) (end 168.779999 95.380001) (width 0.8) (layer F.Cu) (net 55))
 (segment (start 169.507999 115.700001) (end 168.779999 114.972001) (width 0.8) (layer F.Cu) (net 55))
 (segment (start 170.852001 115.700001) (end 169.507999 115.700001) (width 0.8) (layer F.Cu) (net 55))
 (segment (start 174.792002 111.76) (end 170.852001 115.700001) (width 0.8) (layer F.Cu) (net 55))
 (segment (start 175.26 111.76) (end 174.792002 111.76) (width 0.8) (layer F.Cu) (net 55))
 (segment (start 148.720001 114.972001) (end 146.852002 116.84) (width 0.8) (layer F.Cu) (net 54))
 (segment (start 123.122081 116.84) (end 121.92 116.84) (width 0.8) (layer F.Cu) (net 54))
 (segment (start 146.852002 116.84) (end 123.122081 116.84) (width 0.8) (layer F.Cu) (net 54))
 (segment (start 148.720001 110.359999) (end 148.720001 114.972001) (width 0.8) (layer F.Cu) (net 54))
 (segment (start 154.94 104.14) (end 148.720001 110.359999) (width 0.8) (layer F.Cu) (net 54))
 (segment (start 121.070001 117.689999) (end 121.92 116.84) (width 0.8) (layer F.Cu) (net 54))
 (segment (start 103.810009 119.290011) (end 119.469989 119.290011) (width 0.8) (layer F.Cu) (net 54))
 (segment (start 102.689999 118.170001) (end 103.810009 119.290011) (width 0.8) (layer F.Cu) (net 54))
 (segment (start 102.689999 98.363999) (end 102.689999 118.170001) (width 0.8) (layer F.Cu) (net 54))
 (segment (start 119.469989 119.290011) (end 121.070001 117.689999) (width 0.8) (layer F.Cu) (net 54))
 (segment (start 103.443999 97.609999) (end 102.689999 98.363999) (width 0.8) (layer F.Cu) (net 54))
 (segment (start 110.270001 97.609999) (end 103.443999 97.609999) (width 0.8) (layer F.Cu) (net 54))
 (segment (start 116.44 91.44) (end 110.270001 97.609999) (width 0.8) (layer F.Cu) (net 54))
 (segment (start 116.84 91.44) (end 116.44 91.44) (width 0.8) (layer F.Cu) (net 54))
 (segment (start 110.069999 117.689999) (end 109.22 116.84) (width 0.8) (layer B.Cu) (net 53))
 (segment (start 145.402001 118.290001) (end 110.670001 118.290001) (width 0.8) (layer B.Cu) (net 53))
 (segment (start 110.670001 118.290001) (end 110.069999 117.689999) (width 0.8) (layer B.Cu) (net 53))
 (segment (start 153.539999 110.152003) (end 145.402001 118.290001) (width 0.8) (layer B.Cu) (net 53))
 (segment (start 153.539999 103.000001) (end 153.539999 110.152003) (width 0.8) (layer B.Cu) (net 53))
 (segment (start 154.94 101.6) (end 153.539999 103.000001) (width 0.8) (layer B.Cu) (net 53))
 (segment (start 110.069999 115.990001) (end 109.22 116.84) (width 0.8) (layer B.Cu) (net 53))
 (segment (start 110.670001 115.389999) (end 110.069999 115.990001) (width 0.8) (layer B.Cu) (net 53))
 (segment (start 110.670001 104.829999) (end 110.670001 115.389999) (width 0.8) (layer B.Cu) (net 53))
 (segment (start 116.44 99.06) (end 110.670001 104.829999) (width 0.8) (layer B.Cu) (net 53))
 (segment (start 116.84 99.06) (end 116.44 99.06) (width 0.8) (layer B.Cu) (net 53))
 (segment (start 172.72 106.68) (end 175.26 109.22) (width 0.8) (layer F.Cu) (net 56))
 (segment (start 170.18 106.68) (end 172.72 106.68) (width 0.8) (layer F.Cu) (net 56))
 (segment (start 106.68 76.2) (end 106.68 86.36) (width 0.8) (layer F.Cu) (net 37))
 (segment (start 106.68 109.22) (end 106.68 116.84) (width 0.8) (layer B.Cu) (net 37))
 (segment (start 119.38 115.637919) (end 119.38 116.84) (width 0.8) (layer F.Cu) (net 37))
 (segment (start 119.13208 115.389999) (end 119.38 115.637919) (width 0.8) (layer F.Cu) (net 37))
 (segment (start 108.130001 115.389999) (end 119.13208 115.389999) (width 0.8) (layer F.Cu) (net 37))
 (segment (start 106.68 116.84) (end 108.130001 115.389999) (width 0.8) (layer F.Cu) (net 37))
 (segment (start 111.76 104.14) (end 109.22 106.68) (width 0.8) (layer F.Cu) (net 39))
 (segment (start 116.84 104.14) (end 111.76 104.14) (width 0.8) (layer F.Cu) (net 39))
 (segment (start 116.84 96.52) (end 114.3 96.52) (width 0.8) (layer F.Cu) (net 41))
 (segment (start 114.3 96.52) (end 109.22 101.6) (width 0.8) (layer F.Cu) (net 41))
 (segment (start 109.22 76.2) (end 109.22 77.47) (width 0.8) (layer F.Cu) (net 50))
 (segment (start 109.22 77.47) (end 111.76 80.01) (width 0.8) (layer F.Cu) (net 50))
 (segment (start 111.76 88.9) (end 109.22 91.44) (width 0.8) (layer F.Cu) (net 50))
 (segment (start 111.76 80.01) (end 111.76 88.9) (width 0.8) (layer F.Cu) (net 50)))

